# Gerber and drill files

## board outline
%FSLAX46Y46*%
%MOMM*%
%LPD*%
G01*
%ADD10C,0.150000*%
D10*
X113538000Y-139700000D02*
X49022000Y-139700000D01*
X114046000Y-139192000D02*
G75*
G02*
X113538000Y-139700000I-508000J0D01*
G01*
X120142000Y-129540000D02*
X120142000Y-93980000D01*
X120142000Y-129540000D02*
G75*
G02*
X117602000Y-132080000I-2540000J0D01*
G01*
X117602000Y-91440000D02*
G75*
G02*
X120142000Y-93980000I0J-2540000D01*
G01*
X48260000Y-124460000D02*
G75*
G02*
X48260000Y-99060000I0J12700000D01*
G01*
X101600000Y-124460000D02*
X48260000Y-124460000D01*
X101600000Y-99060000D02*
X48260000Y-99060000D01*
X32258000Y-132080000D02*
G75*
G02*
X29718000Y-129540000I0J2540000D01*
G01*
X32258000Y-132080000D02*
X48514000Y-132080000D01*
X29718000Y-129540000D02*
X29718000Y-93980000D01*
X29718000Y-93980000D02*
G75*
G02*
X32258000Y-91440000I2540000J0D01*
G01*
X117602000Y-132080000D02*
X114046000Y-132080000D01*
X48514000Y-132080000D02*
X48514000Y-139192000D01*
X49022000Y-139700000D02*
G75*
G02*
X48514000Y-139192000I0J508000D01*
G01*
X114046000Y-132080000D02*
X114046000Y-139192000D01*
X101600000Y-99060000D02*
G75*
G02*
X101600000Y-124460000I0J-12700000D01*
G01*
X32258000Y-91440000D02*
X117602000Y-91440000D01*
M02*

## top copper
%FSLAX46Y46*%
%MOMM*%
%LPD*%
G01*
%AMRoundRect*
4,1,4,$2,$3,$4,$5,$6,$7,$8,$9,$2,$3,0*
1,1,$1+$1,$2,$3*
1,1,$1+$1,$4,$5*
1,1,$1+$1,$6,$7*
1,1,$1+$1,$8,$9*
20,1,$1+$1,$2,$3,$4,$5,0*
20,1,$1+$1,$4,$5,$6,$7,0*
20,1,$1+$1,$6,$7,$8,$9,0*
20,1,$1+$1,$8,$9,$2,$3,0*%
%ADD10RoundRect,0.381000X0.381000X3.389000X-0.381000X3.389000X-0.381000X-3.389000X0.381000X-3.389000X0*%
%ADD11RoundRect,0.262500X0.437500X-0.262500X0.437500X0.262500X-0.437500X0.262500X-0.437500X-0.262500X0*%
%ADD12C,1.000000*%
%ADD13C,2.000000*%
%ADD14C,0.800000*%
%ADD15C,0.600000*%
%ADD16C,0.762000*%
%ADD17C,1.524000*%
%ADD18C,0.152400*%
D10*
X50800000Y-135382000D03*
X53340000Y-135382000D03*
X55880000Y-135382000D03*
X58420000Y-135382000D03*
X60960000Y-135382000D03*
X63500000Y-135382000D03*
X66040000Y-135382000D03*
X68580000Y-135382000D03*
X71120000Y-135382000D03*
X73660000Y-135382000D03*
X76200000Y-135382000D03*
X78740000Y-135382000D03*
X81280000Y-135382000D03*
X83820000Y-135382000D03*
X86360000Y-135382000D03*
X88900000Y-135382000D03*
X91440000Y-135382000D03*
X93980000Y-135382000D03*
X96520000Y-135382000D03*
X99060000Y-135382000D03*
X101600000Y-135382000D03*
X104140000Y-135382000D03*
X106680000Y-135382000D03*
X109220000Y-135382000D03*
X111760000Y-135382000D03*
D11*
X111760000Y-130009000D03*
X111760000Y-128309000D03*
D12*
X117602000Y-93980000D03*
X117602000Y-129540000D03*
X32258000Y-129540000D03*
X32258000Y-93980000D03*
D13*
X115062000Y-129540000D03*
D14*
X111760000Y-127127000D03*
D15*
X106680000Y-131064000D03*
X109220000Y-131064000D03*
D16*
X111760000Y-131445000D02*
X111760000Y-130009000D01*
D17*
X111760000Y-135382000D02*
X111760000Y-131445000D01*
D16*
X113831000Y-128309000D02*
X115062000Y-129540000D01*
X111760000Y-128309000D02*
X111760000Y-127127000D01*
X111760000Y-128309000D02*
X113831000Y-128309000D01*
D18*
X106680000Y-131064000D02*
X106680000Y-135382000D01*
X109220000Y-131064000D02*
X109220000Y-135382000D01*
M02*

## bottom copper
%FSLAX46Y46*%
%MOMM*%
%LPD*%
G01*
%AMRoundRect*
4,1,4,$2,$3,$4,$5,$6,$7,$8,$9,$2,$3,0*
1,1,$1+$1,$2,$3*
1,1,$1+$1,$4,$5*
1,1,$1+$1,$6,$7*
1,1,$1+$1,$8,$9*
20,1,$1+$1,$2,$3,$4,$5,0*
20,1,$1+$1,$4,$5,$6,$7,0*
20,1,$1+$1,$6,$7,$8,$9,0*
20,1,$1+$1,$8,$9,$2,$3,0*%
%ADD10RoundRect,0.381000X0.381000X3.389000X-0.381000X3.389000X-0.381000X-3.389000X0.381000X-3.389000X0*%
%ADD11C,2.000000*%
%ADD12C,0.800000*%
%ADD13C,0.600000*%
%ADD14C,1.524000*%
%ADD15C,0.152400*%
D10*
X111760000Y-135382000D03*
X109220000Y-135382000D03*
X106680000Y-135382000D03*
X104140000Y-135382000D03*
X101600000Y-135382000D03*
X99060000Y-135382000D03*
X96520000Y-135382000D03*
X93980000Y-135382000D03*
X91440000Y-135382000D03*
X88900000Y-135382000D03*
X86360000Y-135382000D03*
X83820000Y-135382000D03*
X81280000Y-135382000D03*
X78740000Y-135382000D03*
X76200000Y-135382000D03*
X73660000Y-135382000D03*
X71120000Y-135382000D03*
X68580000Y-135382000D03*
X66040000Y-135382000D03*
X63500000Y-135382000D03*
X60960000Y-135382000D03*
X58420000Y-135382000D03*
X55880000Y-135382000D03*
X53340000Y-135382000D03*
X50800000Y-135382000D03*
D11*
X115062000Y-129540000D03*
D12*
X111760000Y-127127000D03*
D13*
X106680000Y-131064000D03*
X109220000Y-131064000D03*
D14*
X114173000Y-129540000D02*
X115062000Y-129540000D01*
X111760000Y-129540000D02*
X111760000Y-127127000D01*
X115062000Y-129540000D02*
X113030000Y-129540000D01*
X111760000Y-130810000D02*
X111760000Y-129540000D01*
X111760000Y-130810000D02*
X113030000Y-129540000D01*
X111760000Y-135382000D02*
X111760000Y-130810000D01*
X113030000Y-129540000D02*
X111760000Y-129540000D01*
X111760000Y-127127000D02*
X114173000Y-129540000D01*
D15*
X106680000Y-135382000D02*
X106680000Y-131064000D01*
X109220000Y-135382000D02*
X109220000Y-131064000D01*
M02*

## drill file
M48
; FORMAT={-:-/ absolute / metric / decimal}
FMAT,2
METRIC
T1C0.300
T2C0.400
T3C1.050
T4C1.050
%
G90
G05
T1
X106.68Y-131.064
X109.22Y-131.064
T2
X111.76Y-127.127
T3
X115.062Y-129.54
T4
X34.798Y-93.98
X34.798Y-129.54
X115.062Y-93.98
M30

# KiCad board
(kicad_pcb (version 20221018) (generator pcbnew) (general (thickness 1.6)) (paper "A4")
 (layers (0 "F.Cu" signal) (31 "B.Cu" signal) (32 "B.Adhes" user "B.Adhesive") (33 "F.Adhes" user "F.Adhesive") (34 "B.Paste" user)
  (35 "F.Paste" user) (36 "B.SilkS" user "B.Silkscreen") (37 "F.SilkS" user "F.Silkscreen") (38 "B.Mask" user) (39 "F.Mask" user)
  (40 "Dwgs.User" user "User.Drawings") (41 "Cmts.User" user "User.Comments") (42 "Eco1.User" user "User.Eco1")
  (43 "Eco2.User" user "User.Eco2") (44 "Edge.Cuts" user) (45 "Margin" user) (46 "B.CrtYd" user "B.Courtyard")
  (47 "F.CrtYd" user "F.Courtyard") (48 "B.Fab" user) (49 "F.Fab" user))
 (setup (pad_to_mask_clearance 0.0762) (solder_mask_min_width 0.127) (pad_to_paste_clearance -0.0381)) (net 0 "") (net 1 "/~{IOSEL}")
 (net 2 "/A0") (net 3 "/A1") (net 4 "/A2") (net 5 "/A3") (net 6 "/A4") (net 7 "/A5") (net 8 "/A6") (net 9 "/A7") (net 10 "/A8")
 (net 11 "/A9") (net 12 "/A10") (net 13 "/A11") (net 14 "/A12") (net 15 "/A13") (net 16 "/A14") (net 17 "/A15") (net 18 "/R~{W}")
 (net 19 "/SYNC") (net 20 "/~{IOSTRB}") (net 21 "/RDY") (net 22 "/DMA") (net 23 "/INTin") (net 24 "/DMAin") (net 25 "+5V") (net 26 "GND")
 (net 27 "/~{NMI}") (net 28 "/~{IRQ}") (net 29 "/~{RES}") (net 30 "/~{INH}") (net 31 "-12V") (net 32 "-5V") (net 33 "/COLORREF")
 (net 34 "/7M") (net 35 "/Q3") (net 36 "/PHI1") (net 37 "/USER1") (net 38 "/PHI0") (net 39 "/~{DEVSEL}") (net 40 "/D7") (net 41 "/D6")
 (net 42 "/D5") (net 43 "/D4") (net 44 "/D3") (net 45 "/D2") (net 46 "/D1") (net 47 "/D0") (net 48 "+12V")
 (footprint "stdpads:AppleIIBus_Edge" (layer "F.Cu") (at 81.28 135.382)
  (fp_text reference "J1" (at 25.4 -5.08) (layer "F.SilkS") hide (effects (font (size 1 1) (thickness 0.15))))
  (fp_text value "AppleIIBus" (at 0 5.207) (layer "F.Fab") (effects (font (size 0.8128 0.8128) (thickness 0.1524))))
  (pad "1" smd roundrect (at -30.48 0 180) (size 1.524 7.54) (layers "F.Cu" "F.Mask") (roundrect_rratio 0.25) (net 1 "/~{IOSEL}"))
  (pad "2" smd roundrect (at -27.94 0 180) (size 1.524 7.54) (layers "F.Cu" "F.Mask") (roundrect_rratio 0.25) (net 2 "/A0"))
  (pad "3" smd roundrect (at -25.4 0 180) (size 1.524 7.54) (layers "F.Cu" "F.Mask") (roundrect_rratio 0.25) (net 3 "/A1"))
  (pad "4" smd roundrect (at -22.86 0 180) (size 1.524 7.54) (layers "F.Cu" "F.Mask") (roundrect_rratio 0.25) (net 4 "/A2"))
  (pad "5" smd roundrect (at -20.32 0 180) (size 1.524 7.54) (layers "F.Cu" "F.Mask") (roundrect_rratio 0.25) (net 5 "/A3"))
  (pad "6" smd roundrect (at -17.78 0 180) (size 1.524 7.54) (layers "F.Cu" "F.Mask") (roundrect_rratio 0.25) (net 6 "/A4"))
  (pad "7" smd roundrect (at -15.24 0 180) (size 1.524 7.54) (layers "F.Cu" "F.Mask") (roundrect_rratio 0.25) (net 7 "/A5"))
  (pad "8" smd roundrect (at -12.7 0 180) (size 1.524 7.54) (layers "F.Cu" "F.Mask") (roundrect_rratio 0.25) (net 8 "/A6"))
  (pad "9" smd roundrect (at -10.16 0 180) (size 1.524 7.54) (layers "F.Cu" "F.Mask") (roundrect_rratio 0.25) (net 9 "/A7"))
  (pad "10" smd roundrect (at -7.62 0 180) (size 1.524 7.54) (layers "F.Cu" "F.Mask") (roundrect_rratio 0.25) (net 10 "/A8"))
  (pad "11" smd roundrect (at -5.08 0 180) (size 1.524 7.54) (layers "F.Cu" "F.Mask") (roundrect_rratio 0.25) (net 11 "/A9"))
  (pad "12" smd roundrect (at -2.54 0 180) (size 1.524 7.54) (layers "F.Cu" "F.Mask") (roundrect_rratio 0.25) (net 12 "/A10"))
  (pad "13" smd roundrect (at 0 0 180) (size 1.524 7.54) (layers "F.Cu" "F.Mask") (roundrect_rratio 0.25) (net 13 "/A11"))
  (pad "14" smd roundrect (at 2.54 0 180) (size 1.524 7.54) (layers "F.Cu" "F.Mask") (roundrect_rratio 0.25) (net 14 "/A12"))
  (pad "15" smd roundrect (at 5.08 0 180) (size 1.524 7.54) (layers "F.Cu" "F.Mask") (roundrect_rratio 0.25) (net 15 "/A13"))
  (pad "16" smd roundrect (at 7.62 0 180) (size 1.524 7.54) (layers "F.Cu" "F.Mask") (roundrect_rratio 0.25) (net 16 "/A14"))
  (pad "17" smd roundrect (at 10.16 0 180) (size 1.524 7.54) (layers "F.Cu" "F.Mask") (roundrect_rratio 0.25) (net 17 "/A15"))
  (pad "18" smd roundrect (at 12.7 0 180) (size 1.524 7.54) (layers "F.Cu" "F.Mask") (roundrect_rratio 0.25) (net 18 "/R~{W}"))
  (pad "19" smd roundrect (at 15.24 0 180) (size 1.524 7.54) (layers "F.Cu" "F.Mask") (roundrect_rratio 0.25) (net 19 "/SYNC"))
  (pad "20" smd roundrect (at 17.78 0 180) (size 1.524 7.54) (layers "F.Cu" "F.Mask") (roundrect_rratio 0.25) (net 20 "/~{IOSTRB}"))
  (pad "21" smd roundrect (at 20.32 0 180) (size 1.524 7.54) (layers "F.Cu" "F.Mask") (roundrect_rratio 0.25) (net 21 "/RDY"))
  (pad "22" smd roundrect (at 22.86 0 180) (size 1.524 7.54) (layers "F.Cu" "F.Mask") (roundrect_rratio 0.25) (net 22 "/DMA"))
  (pad "23" smd roundrect (at 25.4 0 180) (size 1.524 7.54) (layers "F.Cu" "F.Mask") (roundrect_rratio 0.25) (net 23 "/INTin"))
  (pad "24" smd roundrect (at 27.94 0 180) (size 1.524 7.54) (layers "F.Cu" "F.Mask") (roundrect_rratio 0.25) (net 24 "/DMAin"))
  (pad "25" smd roundrect (at 30.48 0 180) (size 1.524 7.54) (layers "F.Cu" "F.Mask") (roundrect_rratio 0.25) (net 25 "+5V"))
  (pad "26" smd roundrect (at 30.48 0 180) (size 1.524 7.54) (layers "B.Cu" "B.Mask") (roundrect_rratio 0.25) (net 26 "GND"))
  (pad "27" smd roundrect (at 27.94 0 180) (size 1.524 7.54) (layers "B.Cu" "B.Mask") (roundrect_rratio 0.25) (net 24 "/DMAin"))
  (pad "28" smd roundrect (at 25.4 0 180) (size 1.524 7.54) (layers "B.Cu" "B.Mask") (roundrect_rratio 0.25) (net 23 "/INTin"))
  (pad "29" smd roundrect (at 22.86 0 180) (size 1.524 7.54) (layers "B.Cu" "B.Mask") (roundrect_rratio 0.25) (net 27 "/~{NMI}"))
  (pad "30" smd roundrect (at 20.32 0 180) (size 1.524 7.54) (layers "B.Cu" "B.Mask") (roundrect_rratio 0.25) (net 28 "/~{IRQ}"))
  (pad "31" smd roundrect (at 17.78 0 180) (size 1.524 7.54) (layers "B.Cu" "B.Mask") (roundrect_rratio 0.25) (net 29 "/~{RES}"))
  (pad "32" smd roundrect (at 15.24 0 180) (size 1.524 7.54) (layers "B.Cu" "B.Mask") (roundrect_rratio 0.25) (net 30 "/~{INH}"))
  (pad "33" smd roundrect (at 12.7 0 180) (size 1.524 7.54) (layers "B.Cu" "B.Mask") (roundrect_rratio 0.25) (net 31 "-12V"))
  (pad "34" smd roundrect (at 10.16 0 180) (size 1.524 7.54) (layers "B.Cu" "B.Mask") (roundrect_rratio 0.25) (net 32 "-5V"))
  (pad "35" smd roundrect (at 7.62 0 180) (size 1.524 7.54) (layers "B.Cu" "B.Mask") (roundrect_rratio 0.25) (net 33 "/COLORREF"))
  (pad "36" smd roundrect (at 5.08 0 180) (size 1.524 7.54) (layers "B.Cu" "B.Mask") (roundrect_rratio 0.25) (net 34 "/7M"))
  (pad "37" smd roundrect (at 2.54 0 180) (size 1.524 7.54) (layers "B.Cu" "B.Mask") (roundrect_rratio 0.25) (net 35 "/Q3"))
  (pad "38" smd roundrect (at 0 0 180) (size 1.524 7.54) (layers "B.Cu" "B.Mask") (roundrect_rratio 0.25) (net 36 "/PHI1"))
  (pad "39" smd roundrect (at -2.54 0 180) (size 1.524 7.54) (layers "B.Cu" "B.Mask") (roundrect_rratio 0.25) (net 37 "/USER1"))
  (pad "40" smd roundrect (at -5.08 0 180) (size 1.524 7.54) (layers "B.Cu" "B.Mask") (roundrect_rratio 0.25) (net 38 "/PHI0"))
  (pad "41" smd roundrect (at -7.62 0 180) (size 1.524 7.54) (layers "B.Cu" "B.Mask") (roundrect_rratio 0.25) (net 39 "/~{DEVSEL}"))
  (pad "42" smd roundrect (at -10.16 0 180) (size 1.524 7.54) (layers "B.Cu" "B.Mask") (roundrect_rratio 0.25) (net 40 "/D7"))
  (pad "43" smd roundrect (at -12.7 0 180) (size 1.524 7.54) (layers "B.Cu" "B.Mask") (roundrect_rratio 0.25) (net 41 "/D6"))
  (pad "44" smd roundrect (at -15.24 0 180) (size 1.524 7.54) (layers "B.Cu" "B.Mask") (roundrect_rratio 0.25) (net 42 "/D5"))
  (pad "45" smd roundrect (at -17.78 0 180) (size 1.524 7.54) (layers "B.Cu" "B.Mask") (roundrect_rratio 0.25) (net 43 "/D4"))
  (pad "46" smd roundrect (at -20.32 0 180) (size 1.524 7.54) (layers "B.Cu" "B.Mask") (roundrect_rratio 0.25) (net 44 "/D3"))
  (pad "47" smd roundrect (at -22.86 0 180) (size 1.524 7.54) (layers "B.Cu" "B.Mask") (roundrect_rratio 0.25) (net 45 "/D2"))
  (pad "48" smd roundrect (at -25.4 0 180) (size 1.524 7.54) (layers "B.Cu" "B.Mask") (roundrect_rratio 0.25) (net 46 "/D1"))
  (pad "49" smd roundrect (at -27.94 0 180) (size 1.524 7.54) (layers "B.Cu" "B.Mask") (roundrect_rratio 0.25) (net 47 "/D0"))
  (pad "50" smd roundrect (at -30.48 0 180) (size 1.524 7.54) (layers "B.Cu" "B.Mask") (roundrect_rratio 0.25) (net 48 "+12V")))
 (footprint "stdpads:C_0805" (layer "F.Cu") (at 111.76 129.159 90)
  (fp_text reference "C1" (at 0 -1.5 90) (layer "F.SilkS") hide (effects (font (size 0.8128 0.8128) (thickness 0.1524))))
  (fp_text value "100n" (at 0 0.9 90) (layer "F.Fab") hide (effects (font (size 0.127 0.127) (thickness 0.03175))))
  (pad "1" smd roundrect (at -0.85 0 90) (size 1.05 1.4) (layers "F.Cu" "F.Paste" "F.Mask") (roundrect_rratio 0.25) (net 25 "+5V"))
  (pad "2" smd roundrect (at 0.85 0 90) (size 1.05 1.4) (layers "F.Cu" "F.Paste" "F.Mask") (roundrect_rratio 0.25) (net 26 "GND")))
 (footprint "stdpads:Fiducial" (layer "F.Cu") (at 117.602 93.98 -90)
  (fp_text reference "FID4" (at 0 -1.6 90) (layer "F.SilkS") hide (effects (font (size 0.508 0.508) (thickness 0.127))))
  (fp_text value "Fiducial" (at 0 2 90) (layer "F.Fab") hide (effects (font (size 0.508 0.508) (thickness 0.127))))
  (pad "~" smd circle (at 0 0 270) (size 1 1) (layers "F.Cu" "F.Mask") (solder_mask_margin 0.5) (clearance 0.575)))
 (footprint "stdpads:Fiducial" (layer "F.Cu") (at 117.602 129.54)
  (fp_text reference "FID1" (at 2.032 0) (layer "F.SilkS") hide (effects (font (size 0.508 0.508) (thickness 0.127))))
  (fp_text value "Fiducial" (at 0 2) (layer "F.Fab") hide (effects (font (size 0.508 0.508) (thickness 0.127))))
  (pad "~" smd circle (at 0 0) (size 1 1) (layers "F.Cu" "F.Mask") (solder_mask_margin 0.5) (clearance 0.575)))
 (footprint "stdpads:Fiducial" (layer "F.Cu") (at 32.258 129.54 180)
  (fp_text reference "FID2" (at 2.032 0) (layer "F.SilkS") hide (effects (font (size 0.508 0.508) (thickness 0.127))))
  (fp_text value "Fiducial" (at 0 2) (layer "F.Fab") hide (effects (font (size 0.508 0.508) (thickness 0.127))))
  (pad "~" smd circle (at 0 0 180) (size 1 1) (layers "F.Cu" "F.Mask") (solder_mask_margin 0.5) (clearance 0.575)))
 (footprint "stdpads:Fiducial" (layer "F.Cu") (at 32.258 93.98 180)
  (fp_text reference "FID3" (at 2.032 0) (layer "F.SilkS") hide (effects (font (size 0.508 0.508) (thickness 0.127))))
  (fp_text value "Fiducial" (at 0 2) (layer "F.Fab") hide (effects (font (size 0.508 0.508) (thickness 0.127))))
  (pad "~" smd circle (at 0 0 180) (size 1 1) (layers "F.Cu" "F.Mask") (solder_mask_margin 0.5) (clearance 0.575)))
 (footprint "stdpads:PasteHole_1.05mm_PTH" (layer "F.Cu") (at 115.062 129.54) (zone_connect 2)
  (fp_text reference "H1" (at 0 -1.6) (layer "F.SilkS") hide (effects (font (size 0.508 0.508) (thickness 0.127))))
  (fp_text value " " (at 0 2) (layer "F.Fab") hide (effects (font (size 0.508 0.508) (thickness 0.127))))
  (pad "1" thru_hole circle (at 0 0) (size 2 2) (drill 1.05) (layers "*.Cu" "*.Mask") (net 26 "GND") (zone_connect 2)))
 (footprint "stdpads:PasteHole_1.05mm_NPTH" (layer "F.Cu") (at 34.798 129.54 180)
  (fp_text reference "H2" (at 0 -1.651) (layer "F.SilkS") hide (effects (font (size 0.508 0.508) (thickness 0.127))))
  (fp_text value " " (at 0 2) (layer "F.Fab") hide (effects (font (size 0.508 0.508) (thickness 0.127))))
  (pad "" np_thru_hole oval (at 0 0 180) (size 1.05 1.05) (drill 1.05) (layers "*.Cu" "*.Mask")))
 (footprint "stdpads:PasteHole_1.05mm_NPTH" (layer "F.Cu") (at 34.798 93.98 180)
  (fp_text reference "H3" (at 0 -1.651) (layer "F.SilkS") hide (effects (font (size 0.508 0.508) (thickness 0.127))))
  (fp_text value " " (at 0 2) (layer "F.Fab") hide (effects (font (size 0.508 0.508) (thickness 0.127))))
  (pad "" np_thru_hole oval (at 0 0 180) (size 1.05 1.05) (drill 1.05) (layers "*.Cu" "*.Mask")))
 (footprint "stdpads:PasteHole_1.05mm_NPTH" (layer "F.Cu") (at 115.062 93.98 -90)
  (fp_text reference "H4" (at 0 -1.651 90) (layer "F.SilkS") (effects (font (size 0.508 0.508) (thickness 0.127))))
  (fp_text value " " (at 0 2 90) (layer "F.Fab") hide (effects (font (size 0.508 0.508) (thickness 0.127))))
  (pad "" np_thru_hole oval (at 0 0 270) (size 1.05 1.05) (drill 1.05) (layers "*.Cu" "*.Mask")))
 (gr_line (start 113.538 139.7) (end 49.022 139.7) (stroke (width 0.15) (type solid)) (layer "Edge.Cuts"))
 (gr_arc (start 114.046 139.192) (mid 113.89721 139.55121) (end 113.538 139.7) (stroke (width 0.15) (type solid)) (layer "Edge.Cuts"))
 (gr_line (start 120.142 129.54) (end 120.142 93.98) (stroke (width 0.15) (type solid)) (layer "Edge.Cuts"))
 (gr_arc (start 120.142 129.54) (mid 119.398051 131.336051) (end 117.602 132.08) (stroke (width 0.15) (type solid)) (layer "Edge.Cuts"))
 (gr_arc (start 117.602 91.44) (mid 119.398051 92.183949) (end 120.142 93.98) (stroke (width 0.15) (type solid)) (layer "Edge.Cuts"))
 (gr_arc (start 48.26 124.46) (mid 35.56 111.76) (end 48.26 99.06) (stroke (width 0.15) (type solid)) (layer "Edge.Cuts"))
 (gr_line (start 101.6 124.46) (end 48.26 124.46) (stroke (width 0.15) (type solid)) (layer "Edge.Cuts"))
 (gr_line (start 101.6 99.06) (end 48.26 99.06) (stroke (width 0.15) (type solid)) (layer "Edge.Cuts"))
 (gr_arc (start 32.258 132.08) (mid 30.461949 131.336051) (end 29.718 129.54) (stroke (width 0.15) (type solid)) (layer "Edge.Cuts"))
 (gr_line (start 32.258 132.08) (end 48.514 132.08) (stroke (width 0.15) (type solid)) (layer "Edge.Cuts"))
 (gr_line (start 29.718 129.54) (end 29.718 93.98) (stroke (width 0.15) (type solid)) (layer "Edge.Cuts"))
 (gr_arc (start 29.718 93.98) (mid 30.461949 92.183949) (end 32.258 91.44) (stroke (width 0.15) (type solid)) (layer "Edge.Cuts"))
 (gr_line (start 117.602 132.08) (end 114.046 132.08) (stroke (width 0.15) (type solid)) (layer "Edge.Cuts"))
 (gr_line (start 48.514 132.08) (end 48.514 139.192) (stroke (width 0.15) (type solid)) (layer "Edge.Cuts"))
 (gr_arc (start 49.022 139.7) (mid 48.66279 139.55121) (end 48.514 139.192) (stroke (width 0.15) (type solid)) (layer "Edge.Cuts"))
 (gr_line (start 114.046 132.08) (end 114.046 139.192) (stroke (width 0.15) (type solid)) (layer "Edge.Cuts"))
 (gr_arc (start 101.6 99.06) (mid 114.3 111.76) (end 101.6 124.46) (stroke (width 0.15) (type solid)) (layer "Edge.Cuts"))
 (gr_line (start 32.258 91.44) (end 117.602 91.44) (stroke (width 0.15) (type solid)) (layer "Edge.Cuts"))
 (segment (start 111.76 131.445) (end 111.76 130.009) (width 0.762) (layer "F.Cu") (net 25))
 (segment (start 111.76 135.382) (end 111.76 131.445) (width 1.524) (layer "F.Cu") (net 25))
 (segment (start 113.831 128.309) (end 115.062 129.54) (width 0.762) (layer "F.Cu") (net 26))
 (segment (start 111.76 128.309) (end 111.76 127.127) (width 0.762) (layer "F.Cu") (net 26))
 (segment (start 111.76 128.309) (end 113.831 128.309) (width 0.762) (layer "F.Cu") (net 26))
 (via (at 111.76 127.127) (size 0.8) (drill 0.4) (layers "F.Cu" "B.Cu") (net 26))
 (segment (start 114.173 129.54) (end 115.062 129.54) (width 1.524) (layer "B.Cu") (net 26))
 (segment (start 111.76 129.54) (end 111.76 127.127) (width 1.524) (layer "B.Cu") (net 26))
 (segment (start 115.062 129.54) (end 113.03 129.54) (width 1.524) (layer "B.Cu") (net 26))
 (segment (start 111.76 130.81) (end 111.76 129.54) (width 1.524) (layer "B.Cu") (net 26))
 (segment (start 111.76 130.81) (end 113.03 129.54) (width 1.524) (layer "B.Cu") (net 26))
 (segment (start 111.76 135.382) (end 111.76 130.81) (width 1.524) (layer "B.Cu") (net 26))
 (segment (start 113.03 129.54) (end 111.76 129.54) (width 1.524) (layer "B.Cu") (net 26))
 (segment (start 111.76 127.127) (end 114.173 129.54) (width 1.524) (layer "B.Cu") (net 26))
 (segment (start 106.68 131.064) (end 106.68 135.382) (width 0.1524) (layer "F.Cu") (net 23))
 (via (at 106.68 131.064) (size 0.6) (drill 0.3) (layers "F.Cu" "B.Cu") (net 23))
 (segment (start 106.68 135.382) (end 106.68 131.064) (width 0.1524) (layer "B.Cu") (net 23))
 (segment (start 109.22 131.064) (end 109.22 135.382) (width 0.1524) (layer "F.Cu") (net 24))
 (via (at 109.22 131.064) (size 0.6) (drill 0.3) (layers "F.Cu" "B.Cu") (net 24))
 (segment (start 109.22 135.382) (end 109.22 131.064) (width 0.1524) (layer "B.Cu") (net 24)))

